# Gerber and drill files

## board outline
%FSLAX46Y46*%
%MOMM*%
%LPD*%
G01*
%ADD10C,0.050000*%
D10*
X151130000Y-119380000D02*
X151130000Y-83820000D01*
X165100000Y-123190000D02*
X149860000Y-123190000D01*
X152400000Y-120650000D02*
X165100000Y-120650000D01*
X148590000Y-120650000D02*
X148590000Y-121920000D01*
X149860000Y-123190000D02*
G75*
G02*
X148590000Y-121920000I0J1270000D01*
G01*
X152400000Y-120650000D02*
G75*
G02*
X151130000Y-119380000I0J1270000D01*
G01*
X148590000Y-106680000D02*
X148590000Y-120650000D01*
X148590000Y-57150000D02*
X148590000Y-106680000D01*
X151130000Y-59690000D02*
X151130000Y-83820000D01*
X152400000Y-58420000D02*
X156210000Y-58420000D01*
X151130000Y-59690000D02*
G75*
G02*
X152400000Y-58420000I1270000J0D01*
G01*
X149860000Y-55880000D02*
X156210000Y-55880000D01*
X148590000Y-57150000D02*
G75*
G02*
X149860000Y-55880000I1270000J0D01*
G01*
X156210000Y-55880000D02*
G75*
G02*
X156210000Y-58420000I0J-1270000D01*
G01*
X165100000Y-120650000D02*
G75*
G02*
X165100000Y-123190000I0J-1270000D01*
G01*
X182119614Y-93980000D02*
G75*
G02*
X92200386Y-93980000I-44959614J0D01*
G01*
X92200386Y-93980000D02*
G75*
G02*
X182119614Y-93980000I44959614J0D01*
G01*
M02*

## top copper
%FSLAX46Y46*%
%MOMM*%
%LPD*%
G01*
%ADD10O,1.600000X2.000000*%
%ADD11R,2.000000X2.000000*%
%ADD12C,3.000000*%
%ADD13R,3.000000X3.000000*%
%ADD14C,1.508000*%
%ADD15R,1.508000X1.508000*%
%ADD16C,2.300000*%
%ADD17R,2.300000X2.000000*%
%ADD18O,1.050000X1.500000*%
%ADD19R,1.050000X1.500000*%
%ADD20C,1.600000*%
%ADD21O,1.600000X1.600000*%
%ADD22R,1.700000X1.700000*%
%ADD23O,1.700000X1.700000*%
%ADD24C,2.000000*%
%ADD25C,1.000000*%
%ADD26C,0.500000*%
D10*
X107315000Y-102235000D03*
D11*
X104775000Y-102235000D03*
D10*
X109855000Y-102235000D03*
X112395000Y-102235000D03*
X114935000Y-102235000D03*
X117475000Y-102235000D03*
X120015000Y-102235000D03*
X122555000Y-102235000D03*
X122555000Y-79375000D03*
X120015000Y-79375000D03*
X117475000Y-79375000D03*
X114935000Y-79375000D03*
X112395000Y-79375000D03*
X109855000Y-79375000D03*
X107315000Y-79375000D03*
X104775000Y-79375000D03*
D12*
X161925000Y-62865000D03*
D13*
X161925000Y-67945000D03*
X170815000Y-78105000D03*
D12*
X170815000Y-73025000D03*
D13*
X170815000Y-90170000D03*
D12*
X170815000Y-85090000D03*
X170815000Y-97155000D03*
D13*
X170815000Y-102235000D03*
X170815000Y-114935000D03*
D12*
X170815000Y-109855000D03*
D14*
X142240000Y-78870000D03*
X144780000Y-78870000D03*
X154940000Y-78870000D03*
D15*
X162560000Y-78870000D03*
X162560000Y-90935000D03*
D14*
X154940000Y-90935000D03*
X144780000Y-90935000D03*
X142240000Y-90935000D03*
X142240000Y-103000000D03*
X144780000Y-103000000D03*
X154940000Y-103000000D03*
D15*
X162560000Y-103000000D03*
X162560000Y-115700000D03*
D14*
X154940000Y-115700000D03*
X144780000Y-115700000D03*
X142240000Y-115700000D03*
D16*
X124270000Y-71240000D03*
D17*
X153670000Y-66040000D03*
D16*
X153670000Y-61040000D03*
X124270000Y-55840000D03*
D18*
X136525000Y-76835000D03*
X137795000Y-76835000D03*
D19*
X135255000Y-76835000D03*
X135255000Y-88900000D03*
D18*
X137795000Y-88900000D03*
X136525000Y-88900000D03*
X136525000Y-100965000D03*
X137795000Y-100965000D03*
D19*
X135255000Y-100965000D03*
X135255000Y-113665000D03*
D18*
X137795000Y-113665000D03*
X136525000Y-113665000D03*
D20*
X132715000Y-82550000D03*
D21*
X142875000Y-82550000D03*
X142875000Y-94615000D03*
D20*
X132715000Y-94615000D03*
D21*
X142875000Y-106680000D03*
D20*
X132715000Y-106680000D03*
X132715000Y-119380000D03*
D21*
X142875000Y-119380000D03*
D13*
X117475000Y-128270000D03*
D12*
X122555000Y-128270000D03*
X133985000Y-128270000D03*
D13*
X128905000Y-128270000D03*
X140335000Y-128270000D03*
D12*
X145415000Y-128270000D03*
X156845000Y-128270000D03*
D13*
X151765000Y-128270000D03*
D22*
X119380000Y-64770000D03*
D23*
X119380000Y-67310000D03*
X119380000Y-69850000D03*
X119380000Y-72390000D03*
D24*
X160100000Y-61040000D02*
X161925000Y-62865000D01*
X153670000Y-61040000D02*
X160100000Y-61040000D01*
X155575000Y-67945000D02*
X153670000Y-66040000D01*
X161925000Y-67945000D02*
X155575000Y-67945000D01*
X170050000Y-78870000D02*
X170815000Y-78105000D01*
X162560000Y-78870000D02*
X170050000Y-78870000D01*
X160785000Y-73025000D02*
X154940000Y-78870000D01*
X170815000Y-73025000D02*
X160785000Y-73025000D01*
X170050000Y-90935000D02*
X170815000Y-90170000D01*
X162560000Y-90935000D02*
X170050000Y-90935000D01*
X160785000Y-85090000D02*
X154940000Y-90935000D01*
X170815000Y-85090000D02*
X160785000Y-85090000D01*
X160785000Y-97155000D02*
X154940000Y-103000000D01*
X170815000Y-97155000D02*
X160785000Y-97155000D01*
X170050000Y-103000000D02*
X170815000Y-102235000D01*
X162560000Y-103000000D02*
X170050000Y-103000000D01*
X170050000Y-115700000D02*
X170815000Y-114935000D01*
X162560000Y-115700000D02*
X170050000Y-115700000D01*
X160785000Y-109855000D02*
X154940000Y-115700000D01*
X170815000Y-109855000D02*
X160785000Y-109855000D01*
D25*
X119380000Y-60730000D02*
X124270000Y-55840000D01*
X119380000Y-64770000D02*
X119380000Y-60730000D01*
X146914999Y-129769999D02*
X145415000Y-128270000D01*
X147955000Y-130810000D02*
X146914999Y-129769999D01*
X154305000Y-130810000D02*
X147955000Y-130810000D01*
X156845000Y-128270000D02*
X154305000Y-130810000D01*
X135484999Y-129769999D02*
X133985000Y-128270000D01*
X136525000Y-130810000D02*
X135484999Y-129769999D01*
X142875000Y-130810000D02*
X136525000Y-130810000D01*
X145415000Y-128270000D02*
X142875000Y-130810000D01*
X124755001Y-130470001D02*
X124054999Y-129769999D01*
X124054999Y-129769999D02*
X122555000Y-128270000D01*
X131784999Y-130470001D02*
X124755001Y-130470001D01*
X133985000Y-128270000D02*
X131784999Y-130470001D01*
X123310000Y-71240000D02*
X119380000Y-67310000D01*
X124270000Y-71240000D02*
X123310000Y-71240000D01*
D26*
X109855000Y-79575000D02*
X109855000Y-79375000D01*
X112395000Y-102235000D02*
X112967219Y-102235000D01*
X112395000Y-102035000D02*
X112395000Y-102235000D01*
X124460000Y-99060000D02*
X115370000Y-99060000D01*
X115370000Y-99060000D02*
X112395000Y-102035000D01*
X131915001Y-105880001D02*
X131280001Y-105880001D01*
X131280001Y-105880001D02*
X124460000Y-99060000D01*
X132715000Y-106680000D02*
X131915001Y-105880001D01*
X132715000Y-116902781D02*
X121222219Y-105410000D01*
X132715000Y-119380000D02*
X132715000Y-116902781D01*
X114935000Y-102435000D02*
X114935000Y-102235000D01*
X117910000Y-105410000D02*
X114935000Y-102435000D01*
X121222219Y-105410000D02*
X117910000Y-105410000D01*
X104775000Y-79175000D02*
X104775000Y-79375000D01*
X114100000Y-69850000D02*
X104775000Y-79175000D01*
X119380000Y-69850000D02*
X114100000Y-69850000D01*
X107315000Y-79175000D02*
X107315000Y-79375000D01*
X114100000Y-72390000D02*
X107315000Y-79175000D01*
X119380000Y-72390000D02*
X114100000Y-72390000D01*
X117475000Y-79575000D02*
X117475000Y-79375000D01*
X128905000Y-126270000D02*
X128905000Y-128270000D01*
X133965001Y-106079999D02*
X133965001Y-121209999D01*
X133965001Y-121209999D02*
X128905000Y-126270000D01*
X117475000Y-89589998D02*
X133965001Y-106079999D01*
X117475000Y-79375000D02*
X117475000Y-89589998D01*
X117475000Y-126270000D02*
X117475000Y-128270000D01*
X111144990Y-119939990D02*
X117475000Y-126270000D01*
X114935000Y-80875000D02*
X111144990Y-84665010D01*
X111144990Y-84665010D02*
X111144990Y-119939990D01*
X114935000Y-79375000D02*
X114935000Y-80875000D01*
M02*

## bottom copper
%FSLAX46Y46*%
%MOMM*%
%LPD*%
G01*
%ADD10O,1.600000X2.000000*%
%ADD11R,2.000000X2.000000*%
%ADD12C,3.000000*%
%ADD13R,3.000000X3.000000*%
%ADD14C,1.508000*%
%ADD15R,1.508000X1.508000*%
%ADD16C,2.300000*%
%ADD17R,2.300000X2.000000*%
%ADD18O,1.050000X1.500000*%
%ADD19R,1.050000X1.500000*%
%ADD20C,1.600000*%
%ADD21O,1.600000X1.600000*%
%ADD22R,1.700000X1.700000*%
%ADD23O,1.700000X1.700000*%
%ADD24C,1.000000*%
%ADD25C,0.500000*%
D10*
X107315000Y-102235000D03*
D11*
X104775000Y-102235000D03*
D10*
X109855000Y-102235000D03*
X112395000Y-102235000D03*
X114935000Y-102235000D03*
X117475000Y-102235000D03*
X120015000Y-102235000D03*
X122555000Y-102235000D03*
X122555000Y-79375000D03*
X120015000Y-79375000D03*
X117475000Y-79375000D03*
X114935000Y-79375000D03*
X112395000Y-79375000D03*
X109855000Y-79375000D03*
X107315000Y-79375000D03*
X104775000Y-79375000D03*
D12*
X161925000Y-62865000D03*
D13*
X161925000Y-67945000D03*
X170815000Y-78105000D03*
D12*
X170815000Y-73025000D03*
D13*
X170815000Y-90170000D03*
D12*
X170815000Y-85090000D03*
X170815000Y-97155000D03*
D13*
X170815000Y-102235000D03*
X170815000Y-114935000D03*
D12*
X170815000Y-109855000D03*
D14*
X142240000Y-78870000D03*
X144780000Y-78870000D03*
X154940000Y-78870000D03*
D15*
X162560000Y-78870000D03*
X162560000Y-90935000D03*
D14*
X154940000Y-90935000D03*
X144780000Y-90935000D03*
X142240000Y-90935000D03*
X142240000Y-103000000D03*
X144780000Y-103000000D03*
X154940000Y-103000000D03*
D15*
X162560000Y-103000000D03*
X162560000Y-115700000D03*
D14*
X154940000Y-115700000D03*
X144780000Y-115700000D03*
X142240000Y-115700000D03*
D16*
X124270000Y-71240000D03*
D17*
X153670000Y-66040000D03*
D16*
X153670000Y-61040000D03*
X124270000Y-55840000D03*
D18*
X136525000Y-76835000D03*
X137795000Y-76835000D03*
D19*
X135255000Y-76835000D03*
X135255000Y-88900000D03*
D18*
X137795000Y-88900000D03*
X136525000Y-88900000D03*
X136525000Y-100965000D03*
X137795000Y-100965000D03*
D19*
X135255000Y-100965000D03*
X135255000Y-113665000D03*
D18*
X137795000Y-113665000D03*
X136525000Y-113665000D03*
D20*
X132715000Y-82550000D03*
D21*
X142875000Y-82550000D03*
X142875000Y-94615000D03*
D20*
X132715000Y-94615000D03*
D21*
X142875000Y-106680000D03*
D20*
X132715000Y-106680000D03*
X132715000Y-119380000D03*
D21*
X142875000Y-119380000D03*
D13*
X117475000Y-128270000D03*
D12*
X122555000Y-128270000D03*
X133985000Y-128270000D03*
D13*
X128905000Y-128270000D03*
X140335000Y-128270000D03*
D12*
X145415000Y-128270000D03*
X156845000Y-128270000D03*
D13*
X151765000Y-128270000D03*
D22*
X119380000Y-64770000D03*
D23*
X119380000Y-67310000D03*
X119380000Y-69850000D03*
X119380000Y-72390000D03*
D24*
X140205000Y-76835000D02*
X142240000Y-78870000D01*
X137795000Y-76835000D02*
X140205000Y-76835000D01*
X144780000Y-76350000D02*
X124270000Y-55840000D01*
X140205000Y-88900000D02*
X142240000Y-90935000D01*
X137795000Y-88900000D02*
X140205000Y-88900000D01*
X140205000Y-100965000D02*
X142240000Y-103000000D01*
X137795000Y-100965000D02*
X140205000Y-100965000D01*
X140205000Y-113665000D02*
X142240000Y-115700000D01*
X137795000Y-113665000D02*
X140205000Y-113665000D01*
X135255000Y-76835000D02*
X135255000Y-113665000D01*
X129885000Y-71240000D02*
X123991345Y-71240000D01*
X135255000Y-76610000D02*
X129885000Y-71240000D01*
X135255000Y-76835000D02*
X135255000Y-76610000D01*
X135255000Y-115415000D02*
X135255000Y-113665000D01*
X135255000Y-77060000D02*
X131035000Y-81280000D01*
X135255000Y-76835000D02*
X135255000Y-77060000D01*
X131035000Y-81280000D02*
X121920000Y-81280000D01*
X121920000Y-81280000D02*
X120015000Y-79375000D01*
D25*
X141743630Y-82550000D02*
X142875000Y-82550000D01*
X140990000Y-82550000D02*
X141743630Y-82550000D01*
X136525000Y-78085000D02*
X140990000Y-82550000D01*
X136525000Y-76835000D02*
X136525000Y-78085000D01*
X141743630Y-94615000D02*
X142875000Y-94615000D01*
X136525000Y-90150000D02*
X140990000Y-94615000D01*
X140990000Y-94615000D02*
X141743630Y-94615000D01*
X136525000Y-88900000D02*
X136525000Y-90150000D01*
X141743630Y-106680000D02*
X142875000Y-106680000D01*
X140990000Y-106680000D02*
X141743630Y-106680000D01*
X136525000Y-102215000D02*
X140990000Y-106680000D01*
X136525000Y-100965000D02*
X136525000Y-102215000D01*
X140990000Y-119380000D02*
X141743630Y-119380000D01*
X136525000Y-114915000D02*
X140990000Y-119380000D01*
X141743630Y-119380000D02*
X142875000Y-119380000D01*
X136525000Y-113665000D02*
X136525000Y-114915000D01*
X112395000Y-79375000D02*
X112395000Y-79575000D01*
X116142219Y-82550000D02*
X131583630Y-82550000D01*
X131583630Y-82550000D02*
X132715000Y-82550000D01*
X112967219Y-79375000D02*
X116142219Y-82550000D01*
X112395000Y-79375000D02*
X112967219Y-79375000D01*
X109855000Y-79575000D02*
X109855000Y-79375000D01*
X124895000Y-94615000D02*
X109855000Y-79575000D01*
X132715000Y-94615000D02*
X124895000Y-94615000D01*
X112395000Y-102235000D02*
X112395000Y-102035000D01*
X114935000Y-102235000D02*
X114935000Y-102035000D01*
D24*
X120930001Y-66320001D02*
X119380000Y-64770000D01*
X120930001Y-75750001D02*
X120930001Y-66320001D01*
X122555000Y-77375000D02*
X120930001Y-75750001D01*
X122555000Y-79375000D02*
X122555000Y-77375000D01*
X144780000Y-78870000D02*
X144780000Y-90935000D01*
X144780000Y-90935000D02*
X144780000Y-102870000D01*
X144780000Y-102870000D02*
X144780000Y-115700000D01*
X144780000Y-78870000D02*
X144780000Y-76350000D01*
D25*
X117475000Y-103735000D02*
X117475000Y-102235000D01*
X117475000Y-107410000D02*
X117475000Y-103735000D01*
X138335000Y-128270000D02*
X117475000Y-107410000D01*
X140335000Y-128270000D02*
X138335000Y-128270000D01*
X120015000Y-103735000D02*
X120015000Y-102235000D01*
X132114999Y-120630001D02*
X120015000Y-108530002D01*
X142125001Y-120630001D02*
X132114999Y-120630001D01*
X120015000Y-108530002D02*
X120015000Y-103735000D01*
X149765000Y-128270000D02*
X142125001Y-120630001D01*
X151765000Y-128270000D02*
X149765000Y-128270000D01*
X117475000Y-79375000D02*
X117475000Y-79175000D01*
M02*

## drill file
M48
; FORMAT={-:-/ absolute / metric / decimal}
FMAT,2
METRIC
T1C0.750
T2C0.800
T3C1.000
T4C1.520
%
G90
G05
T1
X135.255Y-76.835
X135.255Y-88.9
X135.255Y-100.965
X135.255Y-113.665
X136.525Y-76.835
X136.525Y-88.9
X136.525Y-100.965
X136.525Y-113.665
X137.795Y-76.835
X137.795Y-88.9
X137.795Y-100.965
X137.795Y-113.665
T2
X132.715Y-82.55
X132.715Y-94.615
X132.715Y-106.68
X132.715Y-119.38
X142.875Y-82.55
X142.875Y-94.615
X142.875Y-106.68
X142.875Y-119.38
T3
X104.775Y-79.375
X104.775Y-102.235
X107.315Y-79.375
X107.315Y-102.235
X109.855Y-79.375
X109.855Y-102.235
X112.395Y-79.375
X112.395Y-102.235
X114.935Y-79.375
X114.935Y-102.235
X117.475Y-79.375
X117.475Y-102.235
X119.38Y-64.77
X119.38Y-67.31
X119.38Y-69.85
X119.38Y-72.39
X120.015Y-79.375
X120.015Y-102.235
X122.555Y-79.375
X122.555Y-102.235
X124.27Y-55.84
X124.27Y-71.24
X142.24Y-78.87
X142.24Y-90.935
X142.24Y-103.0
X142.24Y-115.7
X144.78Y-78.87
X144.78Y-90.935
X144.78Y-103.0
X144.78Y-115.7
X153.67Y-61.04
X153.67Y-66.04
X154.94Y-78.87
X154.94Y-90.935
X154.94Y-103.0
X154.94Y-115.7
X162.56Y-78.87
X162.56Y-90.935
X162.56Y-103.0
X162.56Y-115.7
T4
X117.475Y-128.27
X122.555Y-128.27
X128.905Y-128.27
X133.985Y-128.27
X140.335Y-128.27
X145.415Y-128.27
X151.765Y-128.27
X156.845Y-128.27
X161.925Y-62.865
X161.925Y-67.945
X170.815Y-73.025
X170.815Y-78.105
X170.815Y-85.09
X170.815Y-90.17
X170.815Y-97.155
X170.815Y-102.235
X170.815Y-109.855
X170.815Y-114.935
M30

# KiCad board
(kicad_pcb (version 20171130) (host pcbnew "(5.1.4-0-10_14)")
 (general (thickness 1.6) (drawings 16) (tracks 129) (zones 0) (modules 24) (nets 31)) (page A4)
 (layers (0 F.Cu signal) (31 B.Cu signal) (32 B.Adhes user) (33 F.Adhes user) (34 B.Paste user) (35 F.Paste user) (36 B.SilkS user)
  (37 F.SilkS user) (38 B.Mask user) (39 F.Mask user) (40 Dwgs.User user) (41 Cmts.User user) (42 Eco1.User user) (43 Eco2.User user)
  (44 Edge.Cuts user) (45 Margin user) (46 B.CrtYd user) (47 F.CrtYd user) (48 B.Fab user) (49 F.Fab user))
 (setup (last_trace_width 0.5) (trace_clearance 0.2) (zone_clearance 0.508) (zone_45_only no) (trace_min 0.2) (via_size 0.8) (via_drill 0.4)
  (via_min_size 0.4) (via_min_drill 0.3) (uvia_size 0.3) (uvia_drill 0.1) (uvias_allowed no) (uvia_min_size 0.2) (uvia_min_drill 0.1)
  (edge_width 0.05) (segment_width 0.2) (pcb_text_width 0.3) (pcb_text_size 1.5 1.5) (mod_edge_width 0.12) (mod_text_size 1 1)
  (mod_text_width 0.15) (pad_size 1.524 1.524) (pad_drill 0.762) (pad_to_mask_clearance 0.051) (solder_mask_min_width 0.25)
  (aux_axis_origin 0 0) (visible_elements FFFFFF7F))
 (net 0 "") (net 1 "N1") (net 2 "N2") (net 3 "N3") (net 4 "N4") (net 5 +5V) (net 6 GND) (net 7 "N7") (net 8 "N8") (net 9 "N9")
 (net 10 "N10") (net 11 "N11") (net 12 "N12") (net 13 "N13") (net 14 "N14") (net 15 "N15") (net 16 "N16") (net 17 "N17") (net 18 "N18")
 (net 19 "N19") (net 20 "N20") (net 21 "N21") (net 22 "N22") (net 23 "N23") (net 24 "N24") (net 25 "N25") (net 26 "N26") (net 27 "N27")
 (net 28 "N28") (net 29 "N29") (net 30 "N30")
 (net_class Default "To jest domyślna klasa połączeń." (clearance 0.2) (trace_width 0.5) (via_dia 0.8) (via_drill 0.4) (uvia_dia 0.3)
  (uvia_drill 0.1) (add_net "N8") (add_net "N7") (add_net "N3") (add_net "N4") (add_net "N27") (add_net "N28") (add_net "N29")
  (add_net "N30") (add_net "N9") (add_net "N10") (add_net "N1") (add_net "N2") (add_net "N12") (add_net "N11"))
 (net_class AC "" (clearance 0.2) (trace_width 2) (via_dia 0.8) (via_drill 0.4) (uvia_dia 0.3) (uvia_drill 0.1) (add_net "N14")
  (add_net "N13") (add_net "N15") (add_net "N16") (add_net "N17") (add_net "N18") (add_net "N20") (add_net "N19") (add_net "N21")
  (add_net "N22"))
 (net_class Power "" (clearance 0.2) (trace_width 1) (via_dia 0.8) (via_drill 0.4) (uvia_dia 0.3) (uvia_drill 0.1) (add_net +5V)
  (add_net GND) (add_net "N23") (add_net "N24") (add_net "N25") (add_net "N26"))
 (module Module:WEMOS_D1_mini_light (layer F.Cu) (at 104.775 102.235 90)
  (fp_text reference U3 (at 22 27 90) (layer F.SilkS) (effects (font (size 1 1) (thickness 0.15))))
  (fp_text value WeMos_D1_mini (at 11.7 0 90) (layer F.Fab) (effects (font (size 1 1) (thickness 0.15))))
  (pad 2 thru_hole oval (at 0 2.54 90) (size 2 1.6) (drill 1) (layers *.Cu *.Mask))
  (pad 1 thru_hole rect (at 0 0 90) (size 2 2) (drill 1) (layers *.Cu *.Mask))
  (pad 3 thru_hole oval (at 0 5.08 90) (size 2 1.6) (drill 1) (layers *.Cu *.Mask))
  (pad 4 thru_hole oval (at 0 7.62 90) (size 2 1.6) (drill 1) (layers *.Cu *.Mask) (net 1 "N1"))
  (pad 5 thru_hole oval (at 0 10.16 90) (size 2 1.6) (drill 1) (layers *.Cu *.Mask) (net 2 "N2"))
  (pad 6 thru_hole oval (at 0 12.7 90) (size 2 1.6) (drill 1) (layers *.Cu *.Mask) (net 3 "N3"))
  (pad 7 thru_hole oval (at 0 15.24 90) (size 2 1.6) (drill 1) (layers *.Cu *.Mask) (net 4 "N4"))
  (pad 8 thru_hole oval (at 0 17.78 90) (size 2 1.6) (drill 1) (layers *.Cu *.Mask))
  (pad 9 thru_hole oval (at 22.86 17.78 90) (size 2 1.6) (drill 1) (layers *.Cu *.Mask) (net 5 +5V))
  (pad 10 thru_hole oval (at 22.86 15.24 90) (size 2 1.6) (drill 1) (layers *.Cu *.Mask) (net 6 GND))
  (pad 11 thru_hole oval (at 22.86 12.7 90) (size 2 1.6) (drill 1) (layers *.Cu *.Mask) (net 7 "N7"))
  (pad 12 thru_hole oval (at 22.86 10.16 90) (size 2 1.6) (drill 1) (layers *.Cu *.Mask) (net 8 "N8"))
  (pad 13 thru_hole oval (at 22.86 7.62 90) (size 2 1.6) (drill 1) (layers *.Cu *.Mask) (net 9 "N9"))
  (pad 14 thru_hole oval (at 22.86 5.08 90) (size 2 1.6) (drill 1) (layers *.Cu *.Mask) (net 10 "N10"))
  (pad 15 thru_hole oval (at 22.86 2.54 90) (size 2 1.6) (drill 1) (layers *.Cu *.Mask) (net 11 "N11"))
  (pad 16 thru_hole oval (at 22.86 0 90) (size 2 1.6) (drill 1) (layers *.Cu *.Mask) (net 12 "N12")))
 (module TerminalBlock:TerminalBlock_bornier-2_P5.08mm (layer F.Cu) (at 161.925 67.945 90)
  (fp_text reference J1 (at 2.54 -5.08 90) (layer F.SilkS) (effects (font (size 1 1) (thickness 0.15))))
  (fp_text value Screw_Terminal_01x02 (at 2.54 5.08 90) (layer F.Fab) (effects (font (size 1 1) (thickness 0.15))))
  (pad 2 thru_hole circle (at 5.08 0 90) (size 3 3) (drill 1.52) (layers *.Cu *.Mask) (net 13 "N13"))
  (pad 1 thru_hole rect (at 0 0 90) (size 3 3) (drill 1.52) (layers *.Cu *.Mask) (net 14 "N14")))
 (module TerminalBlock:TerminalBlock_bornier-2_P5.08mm (layer F.Cu) (at 170.815 78.105 90)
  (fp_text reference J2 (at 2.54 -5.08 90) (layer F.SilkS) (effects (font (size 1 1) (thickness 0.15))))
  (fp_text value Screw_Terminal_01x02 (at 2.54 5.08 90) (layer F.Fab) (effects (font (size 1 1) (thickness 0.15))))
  (pad 1 thru_hole rect (at 0 0 90) (size 3 3) (drill 1.52) (layers *.Cu *.Mask) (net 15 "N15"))
  (pad 2 thru_hole circle (at 5.08 0 90) (size 3 3) (drill 1.52) (layers *.Cu *.Mask) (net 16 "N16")))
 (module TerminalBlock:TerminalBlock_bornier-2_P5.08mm (layer F.Cu) (at 170.815 90.17 90)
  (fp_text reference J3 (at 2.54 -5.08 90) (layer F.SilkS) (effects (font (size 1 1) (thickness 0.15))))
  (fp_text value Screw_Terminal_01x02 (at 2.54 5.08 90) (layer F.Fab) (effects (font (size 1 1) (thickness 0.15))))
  (pad 1 thru_hole rect (at 0 0 90) (size 3 3) (drill 1.52) (layers *.Cu *.Mask) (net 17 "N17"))
  (pad 2 thru_hole circle (at 5.08 0 90) (size 3 3) (drill 1.52) (layers *.Cu *.Mask) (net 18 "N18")))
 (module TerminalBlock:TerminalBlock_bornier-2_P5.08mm (layer F.Cu) (at 170.815 102.235 90)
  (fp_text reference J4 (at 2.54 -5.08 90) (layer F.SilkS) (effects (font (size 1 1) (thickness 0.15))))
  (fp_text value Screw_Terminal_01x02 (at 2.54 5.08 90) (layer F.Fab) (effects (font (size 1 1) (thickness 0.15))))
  (pad 2 thru_hole circle (at 5.08 0 90) (size 3 3) (drill 1.52) (layers *.Cu *.Mask) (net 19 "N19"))
  (pad 1 thru_hole rect (at 0 0 90) (size 3 3) (drill 1.52) (layers *.Cu *.Mask) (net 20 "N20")))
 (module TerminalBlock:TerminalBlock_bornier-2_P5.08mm (layer F.Cu) (at 170.815 114.935 90)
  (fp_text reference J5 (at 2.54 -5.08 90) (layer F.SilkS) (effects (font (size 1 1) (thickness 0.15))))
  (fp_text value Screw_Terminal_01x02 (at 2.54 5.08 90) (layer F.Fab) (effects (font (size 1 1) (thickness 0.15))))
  (pad 1 thru_hole rect (at 0 0 90) (size 3 3) (drill 1.52) (layers *.Cu *.Mask) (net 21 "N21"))
  (pad 2 thru_hole circle (at 5.08 0 90) (size 3 3) (drill 1.52) (layers *.Cu *.Mask) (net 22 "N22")))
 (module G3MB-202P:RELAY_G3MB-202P (layer F.Cu) (at 152.4 77.47)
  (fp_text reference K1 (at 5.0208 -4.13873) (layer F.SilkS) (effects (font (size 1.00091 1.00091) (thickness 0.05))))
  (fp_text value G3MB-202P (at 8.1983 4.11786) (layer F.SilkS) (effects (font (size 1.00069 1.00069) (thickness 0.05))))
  (pad 4 thru_hole circle (at -10.16 1.4) (size 1.508 1.508) (drill 1) (layers *.Cu *.Mask) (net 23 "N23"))
  (pad 3 thru_hole circle (at -7.62 1.4) (size 1.508 1.508) (drill 1) (layers *.Cu *.Mask) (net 5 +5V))
  (pad 2 thru_hole circle (at 2.54 1.4) (size 1.508 1.508) (drill 1) (layers *.Cu *.Mask) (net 16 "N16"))
  (pad 1 thru_hole rect (at 10.16 1.4) (size 1.508 1.508) (drill 1) (layers *.Cu *.Mask) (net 15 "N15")))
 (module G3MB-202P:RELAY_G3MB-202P (layer F.Cu) (at 152.4 89.535)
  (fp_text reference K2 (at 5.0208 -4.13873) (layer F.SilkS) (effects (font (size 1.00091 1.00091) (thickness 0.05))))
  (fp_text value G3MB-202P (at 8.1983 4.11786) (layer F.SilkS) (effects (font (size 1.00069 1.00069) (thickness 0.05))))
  (pad 1 thru_hole rect (at 10.16 1.4) (size 1.508 1.508) (drill 1) (layers *.Cu *.Mask) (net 17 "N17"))
  (pad 2 thru_hole circle (at 2.54 1.4) (size 1.508 1.508) (drill 1) (layers *.Cu *.Mask) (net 18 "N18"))
  (pad 3 thru_hole circle (at -7.62 1.4) (size 1.508 1.508) (drill 1) (layers *.Cu *.Mask) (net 5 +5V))
  (pad 4 thru_hole circle (at -10.16 1.4) (size 1.508 1.508) (drill 1) (layers *.Cu *.Mask) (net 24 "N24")))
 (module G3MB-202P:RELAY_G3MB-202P (layer F.Cu) (at 152.4 101.6)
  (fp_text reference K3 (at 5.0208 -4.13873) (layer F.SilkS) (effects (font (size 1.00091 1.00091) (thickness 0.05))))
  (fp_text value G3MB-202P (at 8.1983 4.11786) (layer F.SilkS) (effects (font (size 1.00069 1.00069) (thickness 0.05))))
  (pad 4 thru_hole circle (at -10.16 1.4) (size 1.508 1.508) (drill 1) (layers *.Cu *.Mask) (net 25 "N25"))
  (pad 3 thru_hole circle (at -7.62 1.4) (size 1.508 1.508) (drill 1) (layers *.Cu *.Mask) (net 5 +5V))
  (pad 2 thru_hole circle (at 2.54 1.4) (size 1.508 1.508) (drill 1) (layers *.Cu *.Mask) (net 19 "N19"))
  (pad 1 thru_hole rect (at 10.16 1.4) (size 1.508 1.508) (drill 1) (layers *.Cu *.Mask) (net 20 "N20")))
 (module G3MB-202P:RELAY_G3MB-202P (layer F.Cu) (at 152.4 114.3)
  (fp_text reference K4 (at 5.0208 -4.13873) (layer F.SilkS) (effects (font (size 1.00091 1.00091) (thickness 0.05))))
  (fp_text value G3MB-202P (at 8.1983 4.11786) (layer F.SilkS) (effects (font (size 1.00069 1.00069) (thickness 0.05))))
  (pad 1 thru_hole rect (at 10.16 1.4) (size 1.508 1.508) (drill 1) (layers *.Cu *.Mask) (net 21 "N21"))
  (pad 2 thru_hole circle (at 2.54 1.4) (size 1.508 1.508) (drill 1) (layers *.Cu *.Mask) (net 22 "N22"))
  (pad 3 thru_hole circle (at -7.62 1.4) (size 1.508 1.508) (drill 1) (layers *.Cu *.Mask) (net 5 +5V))
  (pad 4 thru_hole circle (at -10.16 1.4) (size 1.508 1.508) (drill 1) (layers *.Cu *.Mask) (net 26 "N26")))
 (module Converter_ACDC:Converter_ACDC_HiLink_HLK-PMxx (layer F.Cu) (at 153.67 66.04 180)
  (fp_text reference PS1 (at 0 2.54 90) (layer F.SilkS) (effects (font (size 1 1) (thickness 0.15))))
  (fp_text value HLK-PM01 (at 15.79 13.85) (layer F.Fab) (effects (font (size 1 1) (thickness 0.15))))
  (pad 3 thru_hole circle (at 29.4 -5.2 180) (size 2.3 2.3) (drill 1) (layers *.Cu *.Mask) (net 6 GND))
  (pad 1 thru_hole rect (at 0 0 180) (size 2.3 2) (drill 1) (layers *.Cu *.Mask) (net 14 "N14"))
  (pad 2 thru_hole circle (at 0 5 180) (size 2.3 2.3) (drill 1) (layers *.Cu *.Mask) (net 13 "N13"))
  (pad 4 thru_hole circle (at 29.4 10.2 180) (size 2.3 2.3) (drill 1) (layers *.Cu *.Mask) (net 5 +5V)))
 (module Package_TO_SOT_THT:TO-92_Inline (layer F.Cu) (at 135.255 76.835)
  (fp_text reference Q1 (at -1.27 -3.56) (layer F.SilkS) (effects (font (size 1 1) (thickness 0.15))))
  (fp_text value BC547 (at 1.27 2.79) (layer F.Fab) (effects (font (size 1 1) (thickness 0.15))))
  (pad 2 thru_hole oval (at 1.27 0) (size 1.05 1.5) (drill 0.75) (layers *.Cu *.Mask) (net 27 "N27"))
  (pad 3 thru_hole oval (at 2.54 0) (size 1.05 1.5) (drill 0.75) (layers *.Cu *.Mask) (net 23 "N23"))
  (pad 1 thru_hole rect (at 0 0) (size 1.05 1.5) (drill 0.75) (layers *.Cu *.Mask) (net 6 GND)))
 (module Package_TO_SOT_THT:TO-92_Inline (layer F.Cu) (at 135.255 88.9)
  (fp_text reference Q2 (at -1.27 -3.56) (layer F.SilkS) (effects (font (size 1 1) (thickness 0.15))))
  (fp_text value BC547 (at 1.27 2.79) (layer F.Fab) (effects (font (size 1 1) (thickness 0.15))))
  (pad 1 thru_hole rect (at 0 0) (size 1.05 1.5) (drill 0.75) (layers *.Cu *.Mask) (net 6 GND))
  (pad 3 thru_hole oval (at 2.54 0) (size 1.05 1.5) (drill 0.75) (layers *.Cu *.Mask) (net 24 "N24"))
  (pad 2 thru_hole oval (at 1.27 0) (size 1.05 1.5) (drill 0.75) (layers *.Cu *.Mask) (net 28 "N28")))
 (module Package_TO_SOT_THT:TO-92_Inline (layer F.Cu) (at 135.255 100.965)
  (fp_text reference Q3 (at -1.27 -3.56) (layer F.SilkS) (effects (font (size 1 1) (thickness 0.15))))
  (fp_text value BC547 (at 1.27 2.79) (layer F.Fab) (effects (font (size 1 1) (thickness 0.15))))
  (pad 2 thru_hole oval (at 1.27 0) (size 1.05 1.5) (drill 0.75) (layers *.Cu *.Mask) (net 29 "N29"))
  (pad 3 thru_hole oval (at 2.54 0) (size 1.05 1.5) (drill 0.75) (layers *.Cu *.Mask) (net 25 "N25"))
  (pad 1 thru_hole rect (at 0 0) (size 1.05 1.5) (drill 0.75) (layers *.Cu *.Mask) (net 6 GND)))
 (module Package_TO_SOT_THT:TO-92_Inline (layer F.Cu) (at 135.255 113.665)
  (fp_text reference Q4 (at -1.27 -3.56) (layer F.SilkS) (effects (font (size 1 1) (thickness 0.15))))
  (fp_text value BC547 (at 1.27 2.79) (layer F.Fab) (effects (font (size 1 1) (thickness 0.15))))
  (pad 1 thru_hole rect (at 0 0) (size 1.05 1.5) (drill 0.75) (layers *.Cu *.Mask) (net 6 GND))
  (pad 3 thru_hole oval (at 2.54 0) (size 1.05 1.5) (drill 0.75) (layers *.Cu *.Mask) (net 26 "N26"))
  (pad 2 thru_hole oval (at 1.27 0) (size 1.05 1.5) (drill 0.75) (layers *.Cu *.Mask) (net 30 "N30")))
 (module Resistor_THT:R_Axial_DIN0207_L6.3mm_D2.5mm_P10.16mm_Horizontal (layer F.Cu) (at 132.715 82.55)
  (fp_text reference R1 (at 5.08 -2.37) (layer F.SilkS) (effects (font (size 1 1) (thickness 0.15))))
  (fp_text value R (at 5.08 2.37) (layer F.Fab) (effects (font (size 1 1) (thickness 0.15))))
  (pad 1 thru_hole circle (at 0 0) (size 1.6 1.6) (drill 0.8) (layers *.Cu *.Mask) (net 9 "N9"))
  (pad 2 thru_hole oval (at 10.16 0) (size 1.6 1.6) (drill 0.8) (layers *.Cu *.Mask) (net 27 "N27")))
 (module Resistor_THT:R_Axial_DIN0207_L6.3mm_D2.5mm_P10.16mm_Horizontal (layer F.Cu) (at 132.715 94.615)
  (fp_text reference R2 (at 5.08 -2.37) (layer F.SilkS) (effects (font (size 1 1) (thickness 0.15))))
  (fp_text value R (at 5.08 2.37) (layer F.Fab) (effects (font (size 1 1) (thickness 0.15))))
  (pad 2 thru_hole oval (at 10.16 0) (size 1.6 1.6) (drill 0.8) (layers *.Cu *.Mask) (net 28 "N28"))
  (pad 1 thru_hole circle (at 0 0) (size 1.6 1.6) (drill 0.8) (layers *.Cu *.Mask) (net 10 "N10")))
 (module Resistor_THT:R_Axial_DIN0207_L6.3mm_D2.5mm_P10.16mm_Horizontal (layer F.Cu) (at 132.715 106.68)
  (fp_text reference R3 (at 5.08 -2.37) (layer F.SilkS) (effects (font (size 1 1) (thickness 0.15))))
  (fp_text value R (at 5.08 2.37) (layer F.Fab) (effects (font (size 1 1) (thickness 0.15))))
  (pad 2 thru_hole oval (at 10.16 0) (size 1.6 1.6) (drill 0.8) (layers *.Cu *.Mask) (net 29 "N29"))
  (pad 1 thru_hole circle (at 0 0) (size 1.6 1.6) (drill 0.8) (layers *.Cu *.Mask) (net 1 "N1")))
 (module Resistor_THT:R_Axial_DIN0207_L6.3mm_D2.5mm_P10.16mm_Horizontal (layer F.Cu) (at 132.715 119.38)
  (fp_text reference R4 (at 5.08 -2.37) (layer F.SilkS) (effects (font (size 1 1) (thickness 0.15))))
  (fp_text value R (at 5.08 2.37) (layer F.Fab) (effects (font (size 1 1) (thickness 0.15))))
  (pad 1 thru_hole circle (at 0 0) (size 1.6 1.6) (drill 0.8) (layers *.Cu *.Mask) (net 2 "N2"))
  (pad 2 thru_hole oval (at 10.16 0) (size 1.6 1.6) (drill 0.8) (layers *.Cu *.Mask) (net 30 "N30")))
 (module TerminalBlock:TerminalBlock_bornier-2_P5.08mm (layer F.Cu) (at 117.475 128.27)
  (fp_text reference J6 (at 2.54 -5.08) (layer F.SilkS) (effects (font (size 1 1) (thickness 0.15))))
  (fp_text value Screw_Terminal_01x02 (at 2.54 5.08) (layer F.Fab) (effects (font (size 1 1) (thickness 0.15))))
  (pad 1 thru_hole rect (at 0 0) (size 3 3) (drill 1.52) (layers *.Cu *.Mask) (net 8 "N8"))
  (pad 2 thru_hole circle (at 5.08 0) (size 3 3) (drill 1.52) (layers *.Cu *.Mask) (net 6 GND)))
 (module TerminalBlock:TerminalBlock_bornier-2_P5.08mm (layer F.Cu) (at 128.905 128.27)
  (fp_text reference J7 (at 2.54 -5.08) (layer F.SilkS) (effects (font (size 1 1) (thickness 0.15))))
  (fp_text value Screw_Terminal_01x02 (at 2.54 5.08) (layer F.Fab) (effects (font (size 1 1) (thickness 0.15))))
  (pad 2 thru_hole circle (at 5.08 0) (size 3 3) (drill 1.52) (layers *.Cu *.Mask) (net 6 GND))
  (pad 1 thru_hole rect (at 0 0) (size 3 3) (drill 1.52) (layers *.Cu *.Mask) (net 7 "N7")))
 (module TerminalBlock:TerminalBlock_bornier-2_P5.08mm (layer F.Cu) (at 140.335 128.27)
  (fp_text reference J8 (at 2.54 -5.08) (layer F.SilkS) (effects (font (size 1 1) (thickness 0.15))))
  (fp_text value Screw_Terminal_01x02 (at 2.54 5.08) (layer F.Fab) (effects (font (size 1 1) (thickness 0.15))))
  (pad 1 thru_hole rect (at 0 0) (size 3 3) (drill 1.52) (layers *.Cu *.Mask) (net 3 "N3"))
  (pad 2 thru_hole circle (at 5.08 0) (size 3 3) (drill 1.52) (layers *.Cu *.Mask) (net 6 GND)))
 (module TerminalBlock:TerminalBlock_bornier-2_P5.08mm (layer F.Cu) (at 151.765 128.27)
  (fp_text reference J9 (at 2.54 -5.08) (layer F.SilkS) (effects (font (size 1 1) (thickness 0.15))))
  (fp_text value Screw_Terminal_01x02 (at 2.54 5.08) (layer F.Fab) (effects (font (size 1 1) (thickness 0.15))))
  (pad 2 thru_hole circle (at 5.08 0) (size 3 3) (drill 1.52) (layers *.Cu *.Mask) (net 6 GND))
  (pad 1 thru_hole rect (at 0 0) (size 3 3) (drill 1.52) (layers *.Cu *.Mask) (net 4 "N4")))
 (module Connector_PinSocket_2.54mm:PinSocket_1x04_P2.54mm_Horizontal (layer F.Cu) (at 119.38 64.77)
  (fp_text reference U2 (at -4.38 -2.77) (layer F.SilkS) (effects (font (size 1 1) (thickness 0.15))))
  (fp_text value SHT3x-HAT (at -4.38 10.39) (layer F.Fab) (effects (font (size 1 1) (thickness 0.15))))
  (pad 1 thru_hole rect (at 0 0) (size 1.7 1.7) (drill 1) (layers *.Cu *.Mask) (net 5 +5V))
  (pad 2 thru_hole oval (at 0 2.54) (size 1.7 1.7) (drill 1) (layers *.Cu *.Mask) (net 6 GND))
  (pad 3 thru_hole oval (at 0 5.08) (size 1.7 1.7) (drill 1) (layers *.Cu *.Mask) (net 12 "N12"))
  (pad 4 thru_hole oval (at 0 7.62) (size 1.7 1.7) (drill 1) (layers *.Cu *.Mask) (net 11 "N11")))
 (gr_line (start 151.13 119.38) (end 151.13 83.82) (layer Edge.Cuts) (width 0.05))
 (gr_line (start 165.1 123.19) (end 149.86 123.19) (layer Edge.Cuts) (width 0.05))
 (gr_line (start 152.4 120.65) (end 165.1 120.65) (layer Edge.Cuts) (width 0.05))
 (gr_line (start 148.59 120.65) (end 148.59 121.92) (layer Edge.Cuts) (width 0.05))
 (gr_arc (start 149.86 121.92) (end 148.59 121.92) (angle -90) (layer Edge.Cuts) (width 0.05))
 (gr_arc (start 152.4 119.38) (end 151.13 119.38) (angle -90) (layer Edge.Cuts) (width 0.05))
 (gr_line (start 148.59 106.68) (end 148.59 120.65) (layer Edge.Cuts) (width 0.05))
 (gr_line (start 148.59 57.15) (end 148.59 106.68) (layer Edge.Cuts) (width 0.05))
 (gr_line (start 151.13 59.69) (end 151.13 83.82) (layer Edge.Cuts) (width 0.05))
 (gr_line (start 152.4 58.42) (end 156.21 58.42) (layer Edge.Cuts) (width 0.05))
 (gr_arc (start 152.4 59.69) (end 152.4 58.42) (angle -90) (layer Edge.Cuts) (width 0.05))
 (gr_line (start 149.86 55.88) (end 156.21 55.88) (layer Edge.Cuts) (width 0.05))
 (gr_arc (start 149.86 57.15) (end 149.86 55.88) (angle -90) (layer Edge.Cuts) (width 0.05))
 (gr_arc (start 156.21 57.15) (end 156.21 58.42) (angle -180) (layer Edge.Cuts) (width 0.05))
 (gr_arc (start 165.1 121.92) (end 165.1 123.19) (angle -180) (layer Edge.Cuts) (width 0.05))
 (gr_circle (center 137.16 93.98) (end 173.355 120.65) (layer Edge.Cuts) (width 0.05))
 (segment (start 160.1 61.04) (end 161.925 62.865) (width 2) (layer F.Cu) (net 13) (status 20))
 (segment (start 153.67 61.04) (end 160.1 61.04) (width 2) (layer F.Cu) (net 13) (status 10))
 (segment (start 155.575 67.945) (end 153.67 66.04) (width 2) (layer F.Cu) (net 14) (status 20))
 (segment (start 161.925 67.945) (end 155.575 67.945) (width 2) (layer F.Cu) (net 14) (status 10))
 (segment (start 170.05 78.87) (end 170.815 78.105) (width 2) (layer F.Cu) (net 15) (status 30))
 (segment (start 162.56 78.87) (end 170.05 78.87) (width 2) (layer F.Cu) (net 15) (status 30))
 (segment (start 160.785 73.025) (end 154.94 78.87) (width 2) (layer F.Cu) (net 16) (status 20))
 (segment (start 170.815 73.025) (end 160.785 73.025) (width 2) (layer F.Cu) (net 16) (status 10))
 (segment (start 170.05 90.935) (end 170.815 90.17) (width 2) (layer F.Cu) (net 17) (status 30))
 (segment (start 162.56 90.935) (end 170.05 90.935) (width 2) (layer F.Cu) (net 17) (status 30))
 (segment (start 160.785 85.09) (end 154.94 90.935) (width 2) (layer F.Cu) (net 18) (status 20))
 (segment (start 170.815 85.09) (end 160.785 85.09) (width 2) (layer F.Cu) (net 18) (status 10))
 (segment (start 160.785 97.155) (end 154.94 103) (width 2) (layer F.Cu) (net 19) (status 20))
 (segment (start 170.815 97.155) (end 160.785 97.155) (width 2) (layer F.Cu) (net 19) (status 10))
 (segment (start 170.05 103) (end 170.815 102.235) (width 2) (layer F.Cu) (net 20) (status 30))
 (segment (start 162.56 103) (end 170.05 103) (width 2) (layer F.Cu) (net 20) (status 30))
 (segment (start 170.05 115.7) (end 170.815 114.935) (width 2) (layer F.Cu) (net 21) (status 30))
 (segment (start 162.56 115.7) (end 170.05 115.7) (width 2) (layer F.Cu) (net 21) (status 30))
 (segment (start 160.785 109.855) (end 154.94 115.7) (width 2) (layer F.Cu) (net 22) (status 20))
 (segment (start 170.815 109.855) (end 160.785 109.855) (width 2) (layer F.Cu) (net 22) (status 10))
 (segment (start 140.205 76.835) (end 142.24 78.87) (width 1) (layer B.Cu) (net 23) (status 20))
 (segment (start 137.795 76.835) (end 140.205 76.835) (width 1) (layer B.Cu) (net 23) (status 10))
 (segment (start 144.78 76.35) (end 124.27 55.84) (width 1) (layer B.Cu) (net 5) (status 20))
 (segment (start 119.38 60.73) (end 124.27 55.84) (width 1) (layer F.Cu) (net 5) (status 20))
 (segment (start 119.38 64.77) (end 119.38 60.73) (width 1) (layer F.Cu) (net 5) (status 10))
 (segment (start 140.205 88.9) (end 142.24 90.935) (width 1) (layer B.Cu) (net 24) (status 20))
 (segment (start 137.795 88.9) (end 140.205 88.9) (width 1) (layer B.Cu) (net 24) (status 10))
 (segment (start 140.205 100.965) (end 142.24 103) (width 1) (layer B.Cu) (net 25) (status 20))
 (segment (start 137.795 100.965) (end 140.205 100.965) (width 1) (layer B.Cu) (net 25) (status 10))
 (segment (start 140.205 113.665) (end 142.24 115.7) (width 1) (layer B.Cu) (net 26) (status 20))
 (segment (start 137.795 113.665) (end 140.205 113.665) (width 1) (layer B.Cu) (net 26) (status 10))
 (segment (start 135.255 76.835) (end 135.255 113.665) (width 1) (layer B.Cu) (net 6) (status 30))
 (segment (start 129.885 71.24) (end 123.991345 71.24) (width 1) (layer B.Cu) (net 6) (status 20))
 (segment (start 135.255 76.61) (end 129.885 71.24) (width 1) (layer B.Cu) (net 6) (status 10))
 (segment (start 135.255 76.835) (end 135.255 76.61) (width 1) (layer B.Cu) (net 6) (status 30))
 (segment (start 135.255 115.415) (end 135.255 113.665) (width 1) (layer B.Cu) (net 6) (status 20))
 (segment (start 135.255 77.06) (end 131.035 81.28) (width 1) (layer B.Cu) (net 6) (status 10))
 (segment (start 135.255 76.835) (end 135.255 77.06) (width 1) (layer B.Cu) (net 6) (status 30))
 (segment (start 131.035 81.28) (end 121.92 81.28) (width 1) (layer B.Cu) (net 6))
 (segment (start 121.92 81.28) (end 120.015 79.375) (width 1) (layer B.Cu) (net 6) (status 20))
 (segment (start 146.914999 129.769999) (end 145.415 128.27) (width 1) (layer F.Cu) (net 6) (status 20))
 (segment (start 147.955 130.81) (end 146.914999 129.769999) (width 1) (layer F.Cu) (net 6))
 (segment (start 154.305 130.81) (end 147.955 130.81) (width 1) (layer F.Cu) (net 6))
 (segment (start 156.845 128.27) (end 154.305 130.81) (width 1) (layer F.Cu) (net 6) (status 10))
 (segment (start 135.484999 129.769999) (end 133.985 128.27) (width 1) (layer F.Cu) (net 6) (status 20))
 (segment (start 136.525 130.81) (end 135.484999 129.769999) (width 1) (layer F.Cu) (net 6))
 (segment (start 142.875 130.81) (end 136.525 130.81) (width 1) (layer F.Cu) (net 6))
 (segment (start 145.415 128.27) (end 142.875 130.81) (width 1) (layer F.Cu) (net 6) (status 10))
 (segment (start 124.755001 130.470001) (end 124.054999 129.769999) (width 1) (layer F.Cu) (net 6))
 (segment (start 124.054999 129.769999) (end 122.555 128.27) (width 1) (layer F.Cu) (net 6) (status 20))
 (segment (start 131.784999 130.470001) (end 124.755001 130.470001) (width 1) (layer F.Cu) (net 6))
 (segment (start 133.985 128.27) (end 131.784999 130.470001) (width 1) (layer F.Cu) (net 6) (status 10))
 (segment (start 123.31 71.24) (end 119.38 67.31) (width 1) (layer F.Cu) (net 6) (status 30))
 (segment (start 124.27 71.24) (end 123.31 71.24) (width 1) (layer F.Cu) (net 6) (status 30))
 (segment (start 141.74363 82.55) (end 142.875 82.55) (width 0.5) (layer B.Cu) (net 27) (status 20))
 (segment (start 140.99 82.55) (end 141.74363 82.55) (width 0.5) (layer B.Cu) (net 27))
 (segment (start 136.525 78.085) (end 140.99 82.55) (width 0.5) (layer B.Cu) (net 27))
 (segment (start 136.525 76.835) (end 136.525 78.085) (width 0.5) (layer B.Cu) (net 27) (status 10))
 (segment (start 141.74363 94.615) (end 142.875 94.615) (width 0.5) (layer B.Cu) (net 28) (status 20))
 (segment (start 136.525 90.15) (end 140.99 94.615) (width 0.5) (layer B.Cu) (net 28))
 (segment (start 140.99 94.615) (end 141.74363 94.615) (width 0.5) (layer B.Cu) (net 28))
 (segment (start 136.525 88.9) (end 136.525 90.15) (width 0.5) (layer B.Cu) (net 28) (status 10))
 (segment (start 141.74363 106.68) (end 142.875 106.68) (width 0.5) (layer B.Cu) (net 29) (status 20))
 (segment (start 140.99 106.68) (end 141.74363 106.68) (width 0.5) (layer B.Cu) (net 29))
 (segment (start 136.525 102.215) (end 140.99 106.68) (width 0.5) (layer B.Cu) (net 29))
 (segment (start 136.525 100.965) (end 136.525 102.215) (width 0.5) (layer B.Cu) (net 29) (status 10))
 (segment (start 140.99 119.38) (end 141.74363 119.38) (width 0.5) (layer B.Cu) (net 30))
 (segment (start 136.525 114.915) (end 140.99 119.38) (width 0.5) (layer B.Cu) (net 30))
 (segment (start 141.74363 119.38) (end 142.875 119.38) (width 0.5) (layer B.Cu) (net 30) (status 20))
 (segment (start 136.525 113.665) (end 136.525 114.915) (width 0.5) (layer B.Cu) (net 30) (status 10))
 (segment (start 112.395 79.375) (end 112.395 79.575) (width 0.5) (layer B.Cu) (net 9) (status 30))
 (segment (start 116.142219 82.55) (end 131.58363 82.55) (width 0.5) (layer B.Cu) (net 9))
 (segment (start 131.58363 82.55) (end 132.715 82.55) (width 0.5) (layer B.Cu) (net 9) (status 20))
 (segment (start 112.967219 79.375) (end 116.142219 82.55) (width 0.5) (layer B.Cu) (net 9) (status 10))
 (segment (start 112.395 79.375) (end 112.967219 79.375) (width 0.5) (layer B.Cu) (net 9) (status 30))
 (segment (start 109.855 79.575) (end 109.855 79.375) (width 0.5) (layer F.Cu) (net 10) (status 30))
 (segment (start 109.855 79.575) (end 109.855 79.375) (width 0.5) (layer B.Cu) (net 10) (status 30))
 (segment (start 124.895 94.615) (end 109.855 79.575) (width 0.5) (layer B.Cu) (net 10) (status 20))
 (segment (start 132.715 94.615) (end 124.895 94.615) (width 0.5) (layer B.Cu) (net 10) (status 10))
 (segment (start 112.395 102.235) (end 112.395 102.035) (width 0.5) (layer B.Cu) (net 1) (status 30))
 (segment (start 114.935 102.235) (end 114.935 102.035) (width 0.5) (layer B.Cu) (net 2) (status 30))
 (segment (start 120.930001 66.320001) (end 119.38 64.77) (width 1) (layer B.Cu) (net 5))
 (segment (start 120.930001 75.750001) (end 120.930001 66.320001) (width 1) (layer B.Cu) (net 5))
 (segment (start 122.555 77.375) (end 120.930001 75.750001) (width 1) (layer B.Cu) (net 5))
 (segment (start 122.555 79.375) (end 122.555 77.375) (width 1) (layer B.Cu) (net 5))
 (segment (start 144.78 78.87) (end 144.78 90.935) (width 1) (layer B.Cu) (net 5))
 (segment (start 144.78 90.935) (end 144.78 102.87) (width 1) (layer B.Cu) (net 5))
 (segment (start 144.78 102.87) (end 144.78 115.7) (width 1) (layer B.Cu) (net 5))
 (segment (start 144.78 78.87) (end 144.78 76.35) (width 1) (layer B.Cu) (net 5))
 (segment (start 112.395 102.235) (end 112.967219 102.235) (width 0.5) (layer F.Cu) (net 1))
 (segment (start 112.395 102.035) (end 112.395 102.235) (width 0.5) (layer F.Cu) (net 1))
 (segment (start 124.46 99.06) (end 115.37 99.06) (width 0.5) (layer F.Cu) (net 1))
 (segment (start 115.37 99.06) (end 112.395 102.035) (width 0.5) (layer F.Cu) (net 1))
 (segment (start 131.915001 105.880001) (end 131.280001 105.880001) (width 0.5) (layer F.Cu) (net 1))
 (segment (start 131.280001 105.880001) (end 124.46 99.06) (width 0.5) (layer F.Cu) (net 1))
 (segment (start 132.715 106.68) (end 131.915001 105.880001) (width 0.5) (layer F.Cu) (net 1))
 (segment (start 132.715 116.902781) (end 121.222219 105.41) (width 0.5) (layer F.Cu) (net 2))
 (segment (start 132.715 119.38) (end 132.715 116.902781) (width 0.5) (layer F.Cu) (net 2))
 (segment (start 114.935 102.435) (end 114.935 102.235) (width 0.5) (layer F.Cu) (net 2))
 (segment (start 117.91 105.41) (end 114.935 102.435) (width 0.5) (layer F.Cu) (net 2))
 (segment (start 121.222219 105.41) (end 117.91 105.41) (width 0.5) (layer F.Cu) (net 2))
 (segment (start 104.775 79.175) (end 104.775 79.375) (width 0.5) (layer F.Cu) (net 12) (status 30))
 (segment (start 114.1 69.85) (end 104.775 79.175) (width 0.5) (layer F.Cu) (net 12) (status 20))
 (segment (start 119.38 69.85) (end 114.1 69.85) (width 0.5) (layer F.Cu) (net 12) (status 10))
 (segment (start 107.315 79.175) (end 107.315 79.375) (width 0.5) (layer F.Cu) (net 11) (status 30))
 (segment (start 114.1 72.39) (end 107.315 79.175) (width 0.5) (layer F.Cu) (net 11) (status 20))
 (segment (start 119.38 72.39) (end 114.1 72.39) (width 0.5) (layer F.Cu) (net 11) (status 10))
 (segment (start 117.475 103.735) (end 117.475 102.235) (width 0.5) (layer B.Cu) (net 3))
 (segment (start 117.475 107.41) (end 117.475 103.735) (width 0.5) (layer B.Cu) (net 3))
 (segment (start 138.335 128.27) (end 117.475 107.41) (width 0.5) (layer B.Cu) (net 3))
 (segment (start 140.335 128.27) (end 138.335 128.27) (width 0.5) (layer B.Cu) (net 3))
 (segment (start 120.015 103.735) (end 120.015 102.235) (width 0.5) (layer B.Cu) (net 4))
 (segment (start 132.114999 120.630001) (end 120.015 108.530002) (width 0.5) (layer B.Cu) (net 4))
 (segment (start 142.125001 120.630001) (end 132.114999 120.630001) (width 0.5) (layer B.Cu) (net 4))
 (segment (start 120.015 108.530002) (end 120.015 103.735) (width 0.5) (layer B.Cu) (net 4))
 (segment (start 149.765 128.27) (end 142.125001 120.630001) (width 0.5) (layer B.Cu) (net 4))
 (segment (start 151.765 128.27) (end 149.765 128.27) (width 0.5) (layer B.Cu) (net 4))
 (segment (start 117.475 79.375) (end 117.475 79.175) (width 0.5) (layer B.Cu) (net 7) (status 30))
 (segment (start 117.475 79.575) (end 117.475 79.375) (width 0.5) (layer F.Cu) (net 7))
 (segment (start 128.905 126.27) (end 128.905 128.27) (width 0.5) (layer F.Cu) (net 7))
 (segment (start 133.965001 106.079999) (end 133.965001 121.209999) (width 0.5) (layer F.Cu) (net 7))
 (segment (start 133.965001 121.209999) (end 128.905 126.27) (width 0.5) (layer F.Cu) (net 7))
 (segment (start 117.475 89.589998) (end 133.965001 106.079999) (width 0.5) (layer F.Cu) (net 7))
 (segment (start 117.475 79.375) (end 117.475 89.589998) (width 0.5) (layer F.Cu) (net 7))
 (segment (start 117.475 126.27) (end 117.475 128.27) (width 0.5) (layer F.Cu) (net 8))
 (segment (start 111.14499 119.93999) (end 117.475 126.27) (width 0.5) (layer F.Cu) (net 8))
 (segment (start 114.935 80.875) (end 111.14499 84.66501) (width 0.5) (layer F.Cu) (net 8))
 (segment (start 111.14499 84.66501) (end 111.14499 119.93999) (width 0.5) (layer F.Cu) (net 8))
 (segment (start 114.935 79.375) (end 114.935 80.875) (width 0.5) (layer F.Cu) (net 8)))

